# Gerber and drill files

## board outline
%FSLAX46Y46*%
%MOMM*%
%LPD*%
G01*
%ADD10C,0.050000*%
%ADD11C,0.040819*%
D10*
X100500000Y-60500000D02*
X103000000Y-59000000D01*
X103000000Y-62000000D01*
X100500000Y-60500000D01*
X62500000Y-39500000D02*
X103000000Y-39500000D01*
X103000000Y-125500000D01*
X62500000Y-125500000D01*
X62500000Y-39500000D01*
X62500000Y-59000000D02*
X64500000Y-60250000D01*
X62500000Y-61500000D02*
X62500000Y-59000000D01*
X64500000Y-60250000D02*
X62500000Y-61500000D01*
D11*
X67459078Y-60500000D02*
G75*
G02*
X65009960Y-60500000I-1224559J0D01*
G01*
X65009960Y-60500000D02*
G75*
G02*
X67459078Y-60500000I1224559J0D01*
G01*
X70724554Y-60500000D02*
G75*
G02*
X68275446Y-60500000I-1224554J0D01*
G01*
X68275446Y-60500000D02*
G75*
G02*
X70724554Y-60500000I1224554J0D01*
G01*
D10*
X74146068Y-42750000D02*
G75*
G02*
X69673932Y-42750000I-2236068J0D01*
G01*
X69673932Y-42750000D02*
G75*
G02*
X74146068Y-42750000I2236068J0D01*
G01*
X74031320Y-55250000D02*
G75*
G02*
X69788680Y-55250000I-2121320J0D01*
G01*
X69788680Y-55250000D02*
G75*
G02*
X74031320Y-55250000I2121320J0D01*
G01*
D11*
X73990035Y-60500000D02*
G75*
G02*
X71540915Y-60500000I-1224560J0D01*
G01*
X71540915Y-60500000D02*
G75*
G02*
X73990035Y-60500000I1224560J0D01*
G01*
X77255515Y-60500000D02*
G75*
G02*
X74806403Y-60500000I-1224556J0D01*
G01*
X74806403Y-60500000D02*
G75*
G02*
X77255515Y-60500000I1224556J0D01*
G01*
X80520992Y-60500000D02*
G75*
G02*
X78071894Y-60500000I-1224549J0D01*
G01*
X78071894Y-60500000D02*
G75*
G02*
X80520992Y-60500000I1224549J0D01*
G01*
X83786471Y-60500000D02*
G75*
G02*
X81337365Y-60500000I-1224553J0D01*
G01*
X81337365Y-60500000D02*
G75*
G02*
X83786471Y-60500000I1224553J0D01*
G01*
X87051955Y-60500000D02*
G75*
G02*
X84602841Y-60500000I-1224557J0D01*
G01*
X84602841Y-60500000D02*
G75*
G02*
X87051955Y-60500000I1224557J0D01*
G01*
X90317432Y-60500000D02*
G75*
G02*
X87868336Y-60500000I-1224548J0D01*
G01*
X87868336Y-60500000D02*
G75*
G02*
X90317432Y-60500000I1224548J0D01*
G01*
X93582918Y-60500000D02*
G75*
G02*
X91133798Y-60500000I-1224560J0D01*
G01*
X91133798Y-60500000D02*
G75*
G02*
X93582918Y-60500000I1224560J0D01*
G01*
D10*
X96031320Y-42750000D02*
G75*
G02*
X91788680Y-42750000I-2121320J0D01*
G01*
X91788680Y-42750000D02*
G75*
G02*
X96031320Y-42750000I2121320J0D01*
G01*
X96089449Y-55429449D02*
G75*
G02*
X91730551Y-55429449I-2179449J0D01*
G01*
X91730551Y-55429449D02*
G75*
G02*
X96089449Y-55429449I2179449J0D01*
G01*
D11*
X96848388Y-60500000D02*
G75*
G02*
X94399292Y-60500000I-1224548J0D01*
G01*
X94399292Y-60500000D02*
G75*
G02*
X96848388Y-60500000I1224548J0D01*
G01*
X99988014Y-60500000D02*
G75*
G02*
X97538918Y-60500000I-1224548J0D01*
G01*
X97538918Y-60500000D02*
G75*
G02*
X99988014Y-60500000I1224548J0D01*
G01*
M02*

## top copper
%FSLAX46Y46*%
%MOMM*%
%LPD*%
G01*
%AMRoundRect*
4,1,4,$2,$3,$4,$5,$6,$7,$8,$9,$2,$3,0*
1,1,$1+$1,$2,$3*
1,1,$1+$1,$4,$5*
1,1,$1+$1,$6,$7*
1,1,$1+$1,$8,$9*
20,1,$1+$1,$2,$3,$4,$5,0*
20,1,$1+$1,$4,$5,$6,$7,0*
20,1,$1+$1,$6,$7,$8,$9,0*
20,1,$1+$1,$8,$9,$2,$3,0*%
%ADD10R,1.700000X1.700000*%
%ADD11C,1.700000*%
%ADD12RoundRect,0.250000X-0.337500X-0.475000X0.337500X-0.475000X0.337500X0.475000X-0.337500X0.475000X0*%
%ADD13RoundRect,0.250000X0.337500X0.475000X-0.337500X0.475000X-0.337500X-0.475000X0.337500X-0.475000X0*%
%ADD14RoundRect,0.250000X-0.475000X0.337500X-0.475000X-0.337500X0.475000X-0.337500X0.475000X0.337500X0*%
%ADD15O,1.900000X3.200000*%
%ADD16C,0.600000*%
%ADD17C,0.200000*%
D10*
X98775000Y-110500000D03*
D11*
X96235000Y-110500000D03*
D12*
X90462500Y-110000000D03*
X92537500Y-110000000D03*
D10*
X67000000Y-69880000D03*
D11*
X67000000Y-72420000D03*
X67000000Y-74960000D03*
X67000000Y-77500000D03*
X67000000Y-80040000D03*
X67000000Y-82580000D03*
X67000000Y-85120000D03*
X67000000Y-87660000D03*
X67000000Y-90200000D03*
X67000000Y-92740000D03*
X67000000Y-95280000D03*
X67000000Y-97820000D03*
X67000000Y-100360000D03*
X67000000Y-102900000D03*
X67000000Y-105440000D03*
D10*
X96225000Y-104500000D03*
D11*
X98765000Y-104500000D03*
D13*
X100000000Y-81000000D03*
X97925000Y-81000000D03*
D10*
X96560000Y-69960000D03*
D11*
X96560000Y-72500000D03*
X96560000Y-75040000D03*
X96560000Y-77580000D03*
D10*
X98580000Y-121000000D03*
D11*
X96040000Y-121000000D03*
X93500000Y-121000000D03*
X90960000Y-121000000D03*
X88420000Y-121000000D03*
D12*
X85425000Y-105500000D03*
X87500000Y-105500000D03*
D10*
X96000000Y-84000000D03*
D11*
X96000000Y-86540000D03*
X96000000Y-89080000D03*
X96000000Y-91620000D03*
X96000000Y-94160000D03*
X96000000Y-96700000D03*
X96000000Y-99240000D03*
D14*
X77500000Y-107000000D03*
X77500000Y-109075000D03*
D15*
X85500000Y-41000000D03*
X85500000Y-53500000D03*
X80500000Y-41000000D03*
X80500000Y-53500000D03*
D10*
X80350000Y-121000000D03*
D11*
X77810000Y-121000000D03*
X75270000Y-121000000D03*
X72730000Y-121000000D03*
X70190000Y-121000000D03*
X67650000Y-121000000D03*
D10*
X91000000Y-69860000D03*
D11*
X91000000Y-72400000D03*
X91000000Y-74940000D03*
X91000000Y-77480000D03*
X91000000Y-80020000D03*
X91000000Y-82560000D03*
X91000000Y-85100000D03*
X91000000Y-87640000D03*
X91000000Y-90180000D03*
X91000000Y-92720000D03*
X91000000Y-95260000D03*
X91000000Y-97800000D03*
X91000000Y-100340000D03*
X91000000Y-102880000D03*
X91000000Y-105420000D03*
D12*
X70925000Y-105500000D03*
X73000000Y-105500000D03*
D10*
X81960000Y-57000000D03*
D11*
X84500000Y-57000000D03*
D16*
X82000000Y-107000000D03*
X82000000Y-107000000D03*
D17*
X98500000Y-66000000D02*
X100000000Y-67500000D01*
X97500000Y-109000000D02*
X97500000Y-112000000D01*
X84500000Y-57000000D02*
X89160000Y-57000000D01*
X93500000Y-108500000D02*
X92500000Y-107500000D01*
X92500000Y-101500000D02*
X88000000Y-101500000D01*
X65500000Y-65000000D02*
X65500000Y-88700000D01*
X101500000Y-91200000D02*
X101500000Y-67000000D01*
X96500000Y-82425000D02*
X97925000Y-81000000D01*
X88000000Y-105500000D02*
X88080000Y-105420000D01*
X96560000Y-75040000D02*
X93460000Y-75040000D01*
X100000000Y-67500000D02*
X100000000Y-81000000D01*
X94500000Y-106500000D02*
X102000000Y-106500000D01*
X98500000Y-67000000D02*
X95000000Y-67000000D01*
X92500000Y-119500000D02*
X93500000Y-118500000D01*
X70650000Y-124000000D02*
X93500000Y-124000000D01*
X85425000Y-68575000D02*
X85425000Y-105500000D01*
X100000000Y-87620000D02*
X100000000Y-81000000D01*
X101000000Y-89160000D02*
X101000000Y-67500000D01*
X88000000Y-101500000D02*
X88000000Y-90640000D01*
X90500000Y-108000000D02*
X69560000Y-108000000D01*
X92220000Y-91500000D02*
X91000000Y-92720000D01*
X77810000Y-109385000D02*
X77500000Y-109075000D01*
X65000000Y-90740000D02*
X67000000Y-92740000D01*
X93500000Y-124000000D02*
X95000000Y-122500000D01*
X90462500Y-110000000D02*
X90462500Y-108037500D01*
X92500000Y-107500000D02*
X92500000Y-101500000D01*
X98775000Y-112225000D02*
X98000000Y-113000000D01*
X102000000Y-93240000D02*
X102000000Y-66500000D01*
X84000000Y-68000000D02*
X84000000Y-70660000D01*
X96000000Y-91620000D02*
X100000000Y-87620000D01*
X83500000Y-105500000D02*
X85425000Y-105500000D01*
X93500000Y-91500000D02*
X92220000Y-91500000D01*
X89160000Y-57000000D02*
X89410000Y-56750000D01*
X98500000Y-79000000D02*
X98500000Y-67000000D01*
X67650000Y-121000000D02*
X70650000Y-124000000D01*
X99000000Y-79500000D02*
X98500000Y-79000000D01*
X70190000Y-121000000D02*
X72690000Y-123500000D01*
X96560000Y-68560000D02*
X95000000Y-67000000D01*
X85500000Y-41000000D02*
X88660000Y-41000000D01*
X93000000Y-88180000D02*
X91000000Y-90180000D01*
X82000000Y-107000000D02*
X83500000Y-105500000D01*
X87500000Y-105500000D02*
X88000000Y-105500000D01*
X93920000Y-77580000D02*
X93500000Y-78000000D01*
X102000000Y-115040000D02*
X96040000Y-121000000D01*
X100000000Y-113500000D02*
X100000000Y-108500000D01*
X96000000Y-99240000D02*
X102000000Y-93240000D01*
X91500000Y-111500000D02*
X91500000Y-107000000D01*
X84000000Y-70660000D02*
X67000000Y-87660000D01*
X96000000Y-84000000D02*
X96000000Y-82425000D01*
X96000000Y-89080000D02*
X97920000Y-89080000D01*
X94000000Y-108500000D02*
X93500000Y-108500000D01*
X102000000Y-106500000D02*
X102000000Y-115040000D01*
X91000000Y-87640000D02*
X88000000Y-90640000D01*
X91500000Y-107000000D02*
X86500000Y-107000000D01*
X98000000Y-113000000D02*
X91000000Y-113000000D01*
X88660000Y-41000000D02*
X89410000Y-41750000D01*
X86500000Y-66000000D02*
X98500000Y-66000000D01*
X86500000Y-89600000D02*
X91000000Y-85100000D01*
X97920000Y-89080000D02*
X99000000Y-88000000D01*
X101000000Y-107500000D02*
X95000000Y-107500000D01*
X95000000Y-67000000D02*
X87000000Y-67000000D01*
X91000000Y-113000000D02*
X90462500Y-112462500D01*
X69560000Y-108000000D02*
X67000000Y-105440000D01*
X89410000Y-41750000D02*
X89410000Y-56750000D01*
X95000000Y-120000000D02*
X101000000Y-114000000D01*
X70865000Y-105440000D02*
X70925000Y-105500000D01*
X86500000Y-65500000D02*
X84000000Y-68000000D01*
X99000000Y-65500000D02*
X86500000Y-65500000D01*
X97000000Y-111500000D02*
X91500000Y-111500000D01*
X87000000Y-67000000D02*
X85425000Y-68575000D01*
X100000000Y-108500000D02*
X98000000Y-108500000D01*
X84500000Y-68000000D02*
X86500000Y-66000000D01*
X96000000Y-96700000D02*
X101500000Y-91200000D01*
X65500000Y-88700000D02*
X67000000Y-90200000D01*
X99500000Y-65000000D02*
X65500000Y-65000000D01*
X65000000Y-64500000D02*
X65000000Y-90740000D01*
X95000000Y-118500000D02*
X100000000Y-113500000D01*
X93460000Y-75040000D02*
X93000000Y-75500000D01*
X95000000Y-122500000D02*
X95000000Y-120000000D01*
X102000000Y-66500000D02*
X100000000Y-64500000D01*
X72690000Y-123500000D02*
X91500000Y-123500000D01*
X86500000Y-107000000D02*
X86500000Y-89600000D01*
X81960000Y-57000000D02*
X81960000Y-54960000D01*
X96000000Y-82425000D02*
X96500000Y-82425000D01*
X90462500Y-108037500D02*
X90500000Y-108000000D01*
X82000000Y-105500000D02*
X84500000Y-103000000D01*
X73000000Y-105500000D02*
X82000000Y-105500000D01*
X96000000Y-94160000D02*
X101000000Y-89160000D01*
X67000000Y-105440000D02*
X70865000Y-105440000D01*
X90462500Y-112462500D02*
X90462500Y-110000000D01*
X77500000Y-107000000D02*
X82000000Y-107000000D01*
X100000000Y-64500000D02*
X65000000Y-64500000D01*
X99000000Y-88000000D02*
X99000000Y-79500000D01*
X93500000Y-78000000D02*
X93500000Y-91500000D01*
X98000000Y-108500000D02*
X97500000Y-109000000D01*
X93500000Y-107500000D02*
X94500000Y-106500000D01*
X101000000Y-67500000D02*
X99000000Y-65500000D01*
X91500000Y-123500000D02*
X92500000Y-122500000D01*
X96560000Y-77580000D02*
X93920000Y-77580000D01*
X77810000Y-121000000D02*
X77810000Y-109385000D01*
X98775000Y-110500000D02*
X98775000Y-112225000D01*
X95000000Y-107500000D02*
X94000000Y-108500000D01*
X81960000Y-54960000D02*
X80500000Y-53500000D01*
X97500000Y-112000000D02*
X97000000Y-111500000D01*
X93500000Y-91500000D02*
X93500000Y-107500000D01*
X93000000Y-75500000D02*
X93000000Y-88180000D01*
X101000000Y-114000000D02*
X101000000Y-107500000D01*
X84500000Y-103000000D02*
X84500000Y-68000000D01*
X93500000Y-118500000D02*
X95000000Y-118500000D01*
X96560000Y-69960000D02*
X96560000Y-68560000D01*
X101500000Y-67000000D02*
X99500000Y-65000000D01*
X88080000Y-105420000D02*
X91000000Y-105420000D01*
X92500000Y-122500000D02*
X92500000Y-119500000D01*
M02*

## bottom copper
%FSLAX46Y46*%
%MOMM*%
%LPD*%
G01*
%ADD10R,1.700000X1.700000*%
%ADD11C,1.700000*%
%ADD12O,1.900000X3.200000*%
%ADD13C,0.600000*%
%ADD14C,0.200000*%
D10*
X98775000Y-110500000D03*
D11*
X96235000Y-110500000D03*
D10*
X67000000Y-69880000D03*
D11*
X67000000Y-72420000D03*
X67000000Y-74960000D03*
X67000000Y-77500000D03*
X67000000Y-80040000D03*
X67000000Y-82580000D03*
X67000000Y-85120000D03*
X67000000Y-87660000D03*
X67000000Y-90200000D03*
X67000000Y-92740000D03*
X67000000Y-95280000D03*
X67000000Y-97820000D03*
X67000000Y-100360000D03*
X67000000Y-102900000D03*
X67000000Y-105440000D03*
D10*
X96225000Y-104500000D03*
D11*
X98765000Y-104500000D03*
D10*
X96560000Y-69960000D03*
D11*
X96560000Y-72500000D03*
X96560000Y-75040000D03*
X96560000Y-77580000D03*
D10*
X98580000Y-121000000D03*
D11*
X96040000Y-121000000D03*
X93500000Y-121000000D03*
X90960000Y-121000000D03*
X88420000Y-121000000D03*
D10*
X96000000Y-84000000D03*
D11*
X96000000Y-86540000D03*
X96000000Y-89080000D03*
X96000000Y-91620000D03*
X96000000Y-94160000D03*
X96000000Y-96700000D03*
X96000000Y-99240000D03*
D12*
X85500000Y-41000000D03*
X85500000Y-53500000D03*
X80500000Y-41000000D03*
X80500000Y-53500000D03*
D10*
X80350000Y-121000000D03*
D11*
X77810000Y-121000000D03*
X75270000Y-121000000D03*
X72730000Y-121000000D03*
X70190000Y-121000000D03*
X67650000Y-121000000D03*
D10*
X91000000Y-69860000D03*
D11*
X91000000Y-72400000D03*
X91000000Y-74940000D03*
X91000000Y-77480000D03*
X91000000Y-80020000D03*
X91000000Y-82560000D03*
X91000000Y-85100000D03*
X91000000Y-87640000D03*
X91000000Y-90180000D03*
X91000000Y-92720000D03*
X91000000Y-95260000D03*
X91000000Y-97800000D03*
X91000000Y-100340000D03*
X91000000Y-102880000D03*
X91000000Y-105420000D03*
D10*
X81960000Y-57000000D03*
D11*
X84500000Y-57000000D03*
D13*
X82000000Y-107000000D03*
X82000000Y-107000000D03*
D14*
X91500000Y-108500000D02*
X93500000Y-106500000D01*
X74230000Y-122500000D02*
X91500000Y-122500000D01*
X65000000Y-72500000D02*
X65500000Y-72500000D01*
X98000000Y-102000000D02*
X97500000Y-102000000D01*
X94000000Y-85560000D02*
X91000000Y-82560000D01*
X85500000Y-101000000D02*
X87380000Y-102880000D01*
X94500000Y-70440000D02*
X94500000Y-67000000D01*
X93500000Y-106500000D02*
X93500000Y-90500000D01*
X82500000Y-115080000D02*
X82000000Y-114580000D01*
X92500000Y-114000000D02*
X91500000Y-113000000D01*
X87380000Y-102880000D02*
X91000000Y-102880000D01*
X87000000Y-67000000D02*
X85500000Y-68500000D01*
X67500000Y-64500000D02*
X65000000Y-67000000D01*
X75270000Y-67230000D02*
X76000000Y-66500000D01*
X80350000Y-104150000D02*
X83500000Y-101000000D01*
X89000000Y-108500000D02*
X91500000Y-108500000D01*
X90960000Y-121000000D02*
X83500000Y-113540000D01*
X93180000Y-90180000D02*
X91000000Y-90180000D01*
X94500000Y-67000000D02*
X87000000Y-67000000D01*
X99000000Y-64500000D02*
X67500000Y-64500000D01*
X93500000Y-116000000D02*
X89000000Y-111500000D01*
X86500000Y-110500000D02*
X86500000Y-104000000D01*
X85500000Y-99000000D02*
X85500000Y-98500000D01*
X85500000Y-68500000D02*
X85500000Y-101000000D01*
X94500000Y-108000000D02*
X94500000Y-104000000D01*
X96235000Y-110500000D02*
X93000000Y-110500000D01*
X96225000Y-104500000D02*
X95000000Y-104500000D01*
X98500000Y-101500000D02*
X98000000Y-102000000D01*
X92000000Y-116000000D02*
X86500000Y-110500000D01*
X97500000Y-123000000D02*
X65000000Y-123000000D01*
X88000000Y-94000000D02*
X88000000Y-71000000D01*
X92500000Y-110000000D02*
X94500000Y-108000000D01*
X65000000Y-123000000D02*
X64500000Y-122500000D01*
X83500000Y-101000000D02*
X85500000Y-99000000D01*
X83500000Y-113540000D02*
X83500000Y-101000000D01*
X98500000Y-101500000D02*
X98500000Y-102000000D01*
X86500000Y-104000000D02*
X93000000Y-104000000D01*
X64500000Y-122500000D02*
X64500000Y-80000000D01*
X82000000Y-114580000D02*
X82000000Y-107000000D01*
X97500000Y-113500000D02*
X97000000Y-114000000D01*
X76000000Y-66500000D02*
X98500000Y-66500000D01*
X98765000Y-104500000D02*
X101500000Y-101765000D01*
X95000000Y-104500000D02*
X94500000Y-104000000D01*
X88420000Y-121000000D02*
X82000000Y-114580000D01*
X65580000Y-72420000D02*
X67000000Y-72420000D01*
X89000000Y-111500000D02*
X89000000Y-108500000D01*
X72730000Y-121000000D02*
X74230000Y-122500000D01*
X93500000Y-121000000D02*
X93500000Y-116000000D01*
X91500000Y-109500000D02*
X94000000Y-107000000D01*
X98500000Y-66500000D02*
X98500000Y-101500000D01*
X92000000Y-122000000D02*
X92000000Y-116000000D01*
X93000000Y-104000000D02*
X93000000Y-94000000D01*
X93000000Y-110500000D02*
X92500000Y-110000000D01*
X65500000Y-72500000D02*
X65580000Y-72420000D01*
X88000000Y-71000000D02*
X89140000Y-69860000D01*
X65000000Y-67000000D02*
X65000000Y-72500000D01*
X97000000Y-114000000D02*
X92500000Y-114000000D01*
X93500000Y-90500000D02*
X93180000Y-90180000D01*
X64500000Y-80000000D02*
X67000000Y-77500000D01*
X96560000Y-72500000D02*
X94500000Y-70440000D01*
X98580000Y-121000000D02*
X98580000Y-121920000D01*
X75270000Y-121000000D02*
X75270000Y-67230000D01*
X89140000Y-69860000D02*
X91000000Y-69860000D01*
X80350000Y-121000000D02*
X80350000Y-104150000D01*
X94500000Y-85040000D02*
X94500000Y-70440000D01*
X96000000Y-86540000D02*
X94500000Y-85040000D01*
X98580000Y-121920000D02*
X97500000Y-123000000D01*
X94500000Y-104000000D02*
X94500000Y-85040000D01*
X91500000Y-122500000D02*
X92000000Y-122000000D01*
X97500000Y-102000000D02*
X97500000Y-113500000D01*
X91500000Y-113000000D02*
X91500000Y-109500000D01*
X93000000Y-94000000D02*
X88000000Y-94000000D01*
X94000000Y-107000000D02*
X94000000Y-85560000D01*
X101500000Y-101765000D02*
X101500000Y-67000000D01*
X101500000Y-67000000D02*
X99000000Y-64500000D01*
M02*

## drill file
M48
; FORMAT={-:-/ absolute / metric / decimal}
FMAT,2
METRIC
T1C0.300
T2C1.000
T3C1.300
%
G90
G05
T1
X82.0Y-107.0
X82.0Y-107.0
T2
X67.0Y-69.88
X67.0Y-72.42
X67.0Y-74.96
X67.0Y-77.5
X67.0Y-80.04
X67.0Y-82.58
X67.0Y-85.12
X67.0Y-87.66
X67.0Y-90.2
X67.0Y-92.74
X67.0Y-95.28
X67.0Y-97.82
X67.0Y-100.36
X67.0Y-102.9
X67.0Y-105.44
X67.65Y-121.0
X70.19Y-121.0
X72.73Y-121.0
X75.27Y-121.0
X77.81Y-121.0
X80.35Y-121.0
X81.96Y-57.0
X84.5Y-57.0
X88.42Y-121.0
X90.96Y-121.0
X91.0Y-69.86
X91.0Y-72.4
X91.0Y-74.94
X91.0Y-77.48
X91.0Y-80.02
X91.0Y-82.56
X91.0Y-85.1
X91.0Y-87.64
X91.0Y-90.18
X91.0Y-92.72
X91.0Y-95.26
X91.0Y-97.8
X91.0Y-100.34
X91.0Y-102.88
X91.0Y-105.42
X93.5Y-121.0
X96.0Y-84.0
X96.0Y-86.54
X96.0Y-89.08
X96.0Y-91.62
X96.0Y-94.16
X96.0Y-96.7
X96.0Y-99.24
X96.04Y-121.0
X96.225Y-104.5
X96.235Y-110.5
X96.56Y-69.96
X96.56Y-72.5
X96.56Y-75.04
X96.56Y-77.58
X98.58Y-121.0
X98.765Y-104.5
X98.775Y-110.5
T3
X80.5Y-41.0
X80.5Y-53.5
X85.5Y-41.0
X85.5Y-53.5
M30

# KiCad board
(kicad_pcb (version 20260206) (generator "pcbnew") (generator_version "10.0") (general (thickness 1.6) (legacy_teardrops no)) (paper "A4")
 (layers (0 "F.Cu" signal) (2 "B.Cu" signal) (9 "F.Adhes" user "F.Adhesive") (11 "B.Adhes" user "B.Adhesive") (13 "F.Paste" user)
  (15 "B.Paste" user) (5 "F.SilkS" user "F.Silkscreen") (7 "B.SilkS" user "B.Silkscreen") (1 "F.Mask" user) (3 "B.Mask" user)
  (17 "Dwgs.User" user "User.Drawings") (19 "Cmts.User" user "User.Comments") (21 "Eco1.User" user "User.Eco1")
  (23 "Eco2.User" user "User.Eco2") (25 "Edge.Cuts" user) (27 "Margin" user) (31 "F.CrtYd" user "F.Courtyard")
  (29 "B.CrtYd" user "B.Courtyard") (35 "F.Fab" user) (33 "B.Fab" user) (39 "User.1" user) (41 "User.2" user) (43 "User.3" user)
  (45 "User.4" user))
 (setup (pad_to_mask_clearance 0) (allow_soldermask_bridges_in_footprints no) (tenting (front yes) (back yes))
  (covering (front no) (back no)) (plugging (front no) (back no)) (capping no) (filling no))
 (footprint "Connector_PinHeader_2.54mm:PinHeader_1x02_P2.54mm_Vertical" (layer "F.Cu") (at 98.775 110.5 -90)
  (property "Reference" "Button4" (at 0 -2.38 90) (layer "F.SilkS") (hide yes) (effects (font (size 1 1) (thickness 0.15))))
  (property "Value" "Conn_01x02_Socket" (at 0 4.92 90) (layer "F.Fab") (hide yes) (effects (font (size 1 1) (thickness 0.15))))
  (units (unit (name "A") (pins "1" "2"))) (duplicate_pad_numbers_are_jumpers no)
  (pad "1" thru_hole rect (at 0 0 270) (size 1.7 1.7) (drill 1) (layers "*.Cu" "*.Mask") (remove_unused_layers no))
  (pad "2" thru_hole circle (at 0 2.54 270) (size 1.7 1.7) (drill 1) (layers "*.Cu" "*.Mask") (remove_unused_layers no)))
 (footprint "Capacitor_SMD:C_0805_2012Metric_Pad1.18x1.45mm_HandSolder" (layer "F.Cu") (at 91.5 110)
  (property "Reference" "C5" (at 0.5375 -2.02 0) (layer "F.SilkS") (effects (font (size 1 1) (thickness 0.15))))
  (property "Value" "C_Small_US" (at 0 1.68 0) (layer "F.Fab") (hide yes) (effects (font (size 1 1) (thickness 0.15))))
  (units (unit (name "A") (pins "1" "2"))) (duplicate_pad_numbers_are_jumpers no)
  (pad "1" smd roundrect (at -1.0375 0) (size 1.175 1.45) (layers "F.Cu" "F.Mask" "F.Paste") (roundrect_rratio 0.212766))
  (pad "2" smd roundrect (at 1.0375 0) (size 1.175 1.45) (layers "F.Cu" "F.Mask" "F.Paste") (roundrect_rratio 0.212766)))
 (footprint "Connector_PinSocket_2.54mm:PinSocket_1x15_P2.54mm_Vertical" (layer "F.Cu") (at 67 69.88)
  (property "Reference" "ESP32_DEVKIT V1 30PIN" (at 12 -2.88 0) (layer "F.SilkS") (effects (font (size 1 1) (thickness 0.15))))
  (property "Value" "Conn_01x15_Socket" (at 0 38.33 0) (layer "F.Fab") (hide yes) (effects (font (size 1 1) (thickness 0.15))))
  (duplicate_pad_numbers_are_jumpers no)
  (pad "1" thru_hole rect (at 0 0) (size 1.7 1.7) (drill 1) (layers "*.Cu" "*.Mask") (remove_unused_layers no))
  (pad "2" thru_hole circle (at 0 2.54) (size 1.7 1.7) (drill 1) (layers "*.Cu" "*.Mask") (remove_unused_layers no))
  (pad "3" thru_hole circle (at 0 5.08) (size 1.7 1.7) (drill 1) (layers "*.Cu" "*.Mask") (remove_unused_layers no))
  (pad "4" thru_hole circle (at 0 7.62) (size 1.7 1.7) (drill 1) (layers "*.Cu" "*.Mask") (remove_unused_layers no))
  (pad "5" thru_hole circle (at 0 10.16) (size 1.7 1.7) (drill 1) (layers "*.Cu" "*.Mask") (remove_unused_layers no))
  (pad "6" thru_hole circle (at 0 12.7) (size 1.7 1.7) (drill 1) (layers "*.Cu" "*.Mask") (remove_unused_layers no))
  (pad "7" thru_hole circle (at 0 15.24) (size 1.7 1.7) (drill 1) (layers "*.Cu" "*.Mask") (remove_unused_layers no))
  (pad "8" thru_hole circle (at 0 17.78) (size 1.7 1.7) (drill 1) (layers "*.Cu" "*.Mask") (remove_unused_layers no))
  (pad "9" thru_hole circle (at 0 20.32) (size 1.7 1.7) (drill 1) (layers "*.Cu" "*.Mask") (remove_unused_layers no))
  (pad "10" thru_hole circle (at 0 22.86) (size 1.7 1.7) (drill 1) (layers "*.Cu" "*.Mask") (remove_unused_layers no))
  (pad "11" thru_hole circle (at 0 25.4) (size 1.7 1.7) (drill 1) (layers "*.Cu" "*.Mask") (remove_unused_layers no))
  (pad "12" thru_hole circle (at 0 27.94) (size 1.7 1.7) (drill 1) (layers "*.Cu" "*.Mask") (remove_unused_layers no))
  (pad "13" thru_hole circle (at 0 30.48) (size 1.7 1.7) (drill 1) (layers "*.Cu" "*.Mask") (remove_unused_layers no))
  (pad "14" thru_hole circle (at 0 33.02) (size 1.7 1.7) (drill 1) (layers "*.Cu" "*.Mask") (remove_unused_layers no))
  (pad "15" thru_hole circle (at 0 35.56) (size 1.7 1.7) (drill 1) (layers "*.Cu" "*.Mask") (remove_unused_layers no)))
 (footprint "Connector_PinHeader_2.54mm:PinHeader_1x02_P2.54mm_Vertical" (layer "F.Cu") (at 96.225 104.5 90)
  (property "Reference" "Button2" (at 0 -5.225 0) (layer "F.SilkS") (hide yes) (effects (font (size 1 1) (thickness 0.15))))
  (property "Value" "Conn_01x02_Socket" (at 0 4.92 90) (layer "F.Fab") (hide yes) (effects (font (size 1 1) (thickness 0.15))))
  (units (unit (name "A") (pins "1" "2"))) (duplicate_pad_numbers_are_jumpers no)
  (pad "1" thru_hole rect (at 0 0 90) (size 1.7 1.7) (drill 1) (layers "*.Cu" "*.Mask") (remove_unused_layers no))
  (pad "2" thru_hole circle (at 0 2.54 90) (size 1.7 1.7) (drill 1) (layers "*.Cu" "*.Mask") (remove_unused_layers no)))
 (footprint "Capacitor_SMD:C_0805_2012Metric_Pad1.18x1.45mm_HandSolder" (layer "F.Cu") (at 98.9625 81 180)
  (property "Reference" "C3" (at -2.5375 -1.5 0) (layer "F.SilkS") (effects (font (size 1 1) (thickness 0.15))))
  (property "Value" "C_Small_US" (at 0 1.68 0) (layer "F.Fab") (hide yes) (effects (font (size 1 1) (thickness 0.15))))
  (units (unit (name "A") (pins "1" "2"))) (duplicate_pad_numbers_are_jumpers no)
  (pad "1" smd roundrect (at -1.0375 0 180) (size 1.175 1.45) (layers "F.Cu" "F.Mask" "F.Paste") (roundrect_rratio 0.212766))
  (pad "2" smd roundrect (at 1.0375 0 180) (size 1.175 1.45) (layers "F.Cu" "F.Mask" "F.Paste") (roundrect_rratio 0.212766)))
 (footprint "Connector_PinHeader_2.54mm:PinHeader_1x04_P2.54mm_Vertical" (layer "F.Cu") (at 96.56 69.96)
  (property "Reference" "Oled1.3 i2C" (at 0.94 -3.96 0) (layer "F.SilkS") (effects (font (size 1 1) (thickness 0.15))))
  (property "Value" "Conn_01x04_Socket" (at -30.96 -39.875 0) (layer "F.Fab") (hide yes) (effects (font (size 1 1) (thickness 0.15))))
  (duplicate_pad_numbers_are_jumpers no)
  (pad "1" thru_hole rect (at 0 0) (size 1.7 1.7) (drill 1) (layers "*.Cu" "*.Mask") (remove_unused_layers no))
  (pad "2" thru_hole circle (at 0 2.54) (size 1.7 1.7) (drill 1) (layers "*.Cu" "*.Mask") (remove_unused_layers no))
  (pad "3" thru_hole circle (at 0 5.08) (size 1.7 1.7) (drill 1) (layers "*.Cu" "*.Mask") (remove_unused_layers no))
  (pad "4" thru_hole circle (at 0 7.62) (size 1.7 1.7) (drill 1) (layers "*.Cu" "*.Mask") (remove_unused_layers no)))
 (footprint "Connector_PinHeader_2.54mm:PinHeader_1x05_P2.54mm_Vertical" (layer "F.Cu") (at 98.58 121 -90)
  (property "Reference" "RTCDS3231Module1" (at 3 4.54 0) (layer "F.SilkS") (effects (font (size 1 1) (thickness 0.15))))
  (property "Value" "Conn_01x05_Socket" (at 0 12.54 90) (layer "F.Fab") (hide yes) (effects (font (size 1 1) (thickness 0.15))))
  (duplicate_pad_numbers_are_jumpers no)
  (pad "1" thru_hole rect (at 0 0 270) (size 1.7 1.7) (drill 1) (layers "*.Cu" "*.Mask") (remove_unused_layers no))
  (pad "2" thru_hole circle (at 0 2.54 270) (size 1.7 1.7) (drill 1) (layers "*.Cu" "*.Mask") (remove_unused_layers no))
  (pad "3" thru_hole circle (at 0 5.08 270) (size 1.7 1.7) (drill 1) (layers "*.Cu" "*.Mask") (remove_unused_layers no))
  (pad "4" thru_hole circle (at 0 7.62 270) (size 1.7 1.7) (drill 1) (layers "*.Cu" "*.Mask") (remove_unused_layers no))
  (pad "5" thru_hole circle (at 0 10.16 270) (size 1.7 1.7) (drill 1) (layers "*.Cu" "*.Mask") (remove_unused_layers no)))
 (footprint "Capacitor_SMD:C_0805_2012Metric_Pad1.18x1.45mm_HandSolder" (layer "F.Cu") (at 86.4625 105.5)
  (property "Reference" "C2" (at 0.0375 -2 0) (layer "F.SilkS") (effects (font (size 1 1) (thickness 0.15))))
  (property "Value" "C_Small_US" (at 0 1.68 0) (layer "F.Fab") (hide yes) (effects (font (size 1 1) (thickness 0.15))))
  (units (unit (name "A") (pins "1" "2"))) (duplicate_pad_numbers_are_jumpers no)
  (pad "1" smd roundrect (at -1.0375 0) (size 1.175 1.45) (layers "F.Cu" "F.Mask" "F.Paste") (roundrect_rratio 0.212766))
  (pad "2" smd roundrect (at 1.0375 0) (size 1.175 1.45) (layers "F.Cu" "F.Mask" "F.Paste") (roundrect_rratio 0.212766)))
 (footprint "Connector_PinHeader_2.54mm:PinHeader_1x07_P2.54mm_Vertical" (layer "F.Cu") (at 96 84)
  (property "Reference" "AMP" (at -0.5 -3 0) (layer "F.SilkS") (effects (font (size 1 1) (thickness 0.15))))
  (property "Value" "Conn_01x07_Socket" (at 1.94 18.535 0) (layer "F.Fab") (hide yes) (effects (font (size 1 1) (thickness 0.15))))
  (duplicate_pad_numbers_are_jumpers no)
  (pad "1" thru_hole rect (at 0 0) (size 1.7 1.7) (drill 1) (layers "*.Cu" "*.Mask") (remove_unused_layers no))
  (pad "2" thru_hole circle (at 0 2.54) (size 1.7 1.7) (drill 1) (layers "*.Cu" "*.Mask") (remove_unused_layers no))
  (pad "3" thru_hole circle (at 0 5.08) (size 1.7 1.7) (drill 1) (layers "*.Cu" "*.Mask") (remove_unused_layers no))
  (pad "4" thru_hole circle (at 0 7.62) (size 1.7 1.7) (drill 1) (layers "*.Cu" "*.Mask") (remove_unused_layers no))
  (pad "5" thru_hole circle (at 0 10.16) (size 1.7 1.7) (drill 1) (layers "*.Cu" "*.Mask") (remove_unused_layers no))
  (pad "6" thru_hole circle (at 0 12.7) (size 1.7 1.7) (drill 1) (layers "*.Cu" "*.Mask") (remove_unused_layers no))
  (pad "7" thru_hole circle (at 0 15.24) (size 1.7 1.7) (drill 1) (layers "*.Cu" "*.Mask") (remove_unused_layers no)))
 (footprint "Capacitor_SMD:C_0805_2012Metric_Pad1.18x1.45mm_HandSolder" (layer "F.Cu") (at 77.5 108.0375 -90)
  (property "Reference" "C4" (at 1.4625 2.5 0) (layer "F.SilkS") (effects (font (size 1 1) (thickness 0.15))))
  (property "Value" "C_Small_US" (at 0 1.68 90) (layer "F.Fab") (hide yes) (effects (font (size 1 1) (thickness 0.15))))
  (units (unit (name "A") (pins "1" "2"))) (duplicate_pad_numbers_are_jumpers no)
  (pad "1" smd roundrect (at -1.0375 0 270) (size 1.175 1.45) (layers "F.Cu" "F.Mask" "F.Paste") (roundrect_rratio 0.212766))
  (pad "2" smd roundrect (at 1.0375 0 270) (size 1.175 1.45) (layers "F.Cu" "F.Mask" "F.Paste") (roundrect_rratio 0.212766)))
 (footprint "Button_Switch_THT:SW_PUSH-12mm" (layer "F.Cu") (at 85.5 41 -90)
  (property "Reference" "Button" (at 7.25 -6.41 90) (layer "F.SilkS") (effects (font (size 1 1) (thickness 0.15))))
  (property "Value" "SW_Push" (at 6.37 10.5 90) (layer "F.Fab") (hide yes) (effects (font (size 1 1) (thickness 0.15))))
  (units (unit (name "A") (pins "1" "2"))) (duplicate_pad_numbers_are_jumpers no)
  (pad "1" thru_hole oval (at 0 0 270) (size 3.2 1.9) (drill 1.3) (layers "*.Cu" "*.Mask") (remove_unused_layers no))
  (pad "1" thru_hole oval (at 12.5 0 270) (size 3.2 1.9) (drill 1.3) (layers "*.Cu" "*.Mask") (remove_unused_layers no))
  (pad "2" thru_hole oval (at 0 5 270) (size 3.2 1.9) (drill 1.3) (layers "*.Cu" "*.Mask") (remove_unused_layers no))
  (pad "2" thru_hole oval (at 12.5 5 270) (size 3.2 1.9) (drill 1.3) (layers "*.Cu" "*.Mask") (remove_unused_layers no)))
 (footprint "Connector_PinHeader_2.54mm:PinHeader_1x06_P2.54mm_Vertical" (layer "F.Cu") (at 80.35 121 -90)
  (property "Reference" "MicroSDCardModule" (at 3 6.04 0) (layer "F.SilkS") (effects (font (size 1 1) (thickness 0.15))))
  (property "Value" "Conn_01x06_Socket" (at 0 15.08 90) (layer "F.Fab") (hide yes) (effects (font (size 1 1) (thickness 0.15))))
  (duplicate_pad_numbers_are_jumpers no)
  (pad "1" thru_hole rect (at 0 0 270) (size 1.7 1.7) (drill 1) (layers "*.Cu" "*.Mask") (remove_unused_layers no))
  (pad "2" thru_hole circle (at 0 2.54 270) (size 1.7 1.7) (drill 1) (layers "*.Cu" "*.Mask") (remove_unused_layers no))
  (pad "3" thru_hole circle (at 0 5.08 270) (size 1.7 1.7) (drill 1) (layers "*.Cu" "*.Mask") (remove_unused_layers no))
  (pad "4" thru_hole circle (at 0 7.62 270) (size 1.7 1.7) (drill 1) (layers "*.Cu" "*.Mask") (remove_unused_layers no))
  (pad "5" thru_hole circle (at 0 10.16 270) (size 1.7 1.7) (drill 1) (layers "*.Cu" "*.Mask") (remove_unused_layers no))
  (pad "6" thru_hole circle (at 0 12.7 270) (size 1.7 1.7) (drill 1) (layers "*.Cu" "*.Mask") (remove_unused_layers no)))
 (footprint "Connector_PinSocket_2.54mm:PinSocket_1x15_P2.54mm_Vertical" (layer "F.Cu") (at 91 69.86)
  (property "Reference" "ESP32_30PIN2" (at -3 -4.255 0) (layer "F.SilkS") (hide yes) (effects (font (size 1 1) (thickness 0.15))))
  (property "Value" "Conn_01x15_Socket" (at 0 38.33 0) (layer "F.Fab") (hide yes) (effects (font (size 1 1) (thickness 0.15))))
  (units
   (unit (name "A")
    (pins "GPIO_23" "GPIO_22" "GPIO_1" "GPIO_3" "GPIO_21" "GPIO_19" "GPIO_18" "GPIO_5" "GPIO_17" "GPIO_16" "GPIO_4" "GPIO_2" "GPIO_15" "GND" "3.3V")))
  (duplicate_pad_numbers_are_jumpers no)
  (pad "1" thru_hole rect (at 0 0) (size 1.7 1.7) (drill 1) (layers "*.Cu" "*.Mask") (remove_unused_layers no))
  (pad "2" thru_hole circle (at 0 2.54) (size 1.7 1.7) (drill 1) (layers "*.Cu" "*.Mask") (remove_unused_layers no))
  (pad "3" thru_hole circle (at 0 5.08) (size 1.7 1.7) (drill 1) (layers "*.Cu" "*.Mask") (remove_unused_layers no))
  (pad "4" thru_hole circle (at 0 7.62) (size 1.7 1.7) (drill 1) (layers "*.Cu" "*.Mask") (remove_unused_layers no))
  (pad "5" thru_hole circle (at 0 10.16) (size 1.7 1.7) (drill 1) (layers "*.Cu" "*.Mask") (remove_unused_layers no))
  (pad "6" thru_hole circle (at 0 12.7) (size 1.7 1.7) (drill 1) (layers "*.Cu" "*.Mask") (remove_unused_layers no))
  (pad "7" thru_hole circle (at 0 15.24) (size 1.7 1.7) (drill 1) (layers "*.Cu" "*.Mask") (remove_unused_layers no))
  (pad "8" thru_hole circle (at 0 17.78) (size 1.7 1.7) (drill 1) (layers "*.Cu" "*.Mask") (remove_unused_layers no))
  (pad "9" thru_hole circle (at 0 20.32) (size 1.7 1.7) (drill 1) (layers "*.Cu" "*.Mask") (remove_unused_layers no))
  (pad "10" thru_hole circle (at 0 22.86) (size 1.7 1.7) (drill 1) (layers "*.Cu" "*.Mask") (remove_unused_layers no))
  (pad "11" thru_hole circle (at 0 25.4) (size 1.7 1.7) (drill 1) (layers "*.Cu" "*.Mask") (remove_unused_layers no))
  (pad "12" thru_hole circle (at 0 27.94) (size 1.7 1.7) (drill 1) (layers "*.Cu" "*.Mask") (remove_unused_layers no))
  (pad "13" thru_hole circle (at 0 30.48) (size 1.7 1.7) (drill 1) (layers "*.Cu" "*.Mask") (remove_unused_layers no))
  (pad "14" thru_hole circle (at 0 33.02) (size 1.7 1.7) (drill 1) (layers "*.Cu" "*.Mask") (remove_unused_layers no))
  (pad "15" thru_hole circle (at 0 35.56) (size 1.7 1.7) (drill 1) (layers "*.Cu" "*.Mask") (remove_unused_layers no)))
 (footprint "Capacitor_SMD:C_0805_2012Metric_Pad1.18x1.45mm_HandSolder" (layer "F.Cu") (at 71.9625 105.5)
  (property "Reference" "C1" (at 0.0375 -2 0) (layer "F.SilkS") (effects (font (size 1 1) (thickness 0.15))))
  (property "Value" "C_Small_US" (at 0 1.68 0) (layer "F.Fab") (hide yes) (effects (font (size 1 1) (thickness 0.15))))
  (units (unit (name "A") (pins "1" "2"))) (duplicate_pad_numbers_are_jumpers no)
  (pad "1" smd roundrect (at -1.0375 0) (size 1.175 1.45) (layers "F.Cu" "F.Mask" "F.Paste") (roundrect_rratio 0.212766))
  (pad "2" smd roundrect (at 1.0375 0) (size 1.175 1.45) (layers "F.Cu" "F.Mask" "F.Paste") (roundrect_rratio 0.212766)))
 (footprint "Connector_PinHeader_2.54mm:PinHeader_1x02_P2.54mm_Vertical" (layer "B.Cu") (at 81.96 57 -90)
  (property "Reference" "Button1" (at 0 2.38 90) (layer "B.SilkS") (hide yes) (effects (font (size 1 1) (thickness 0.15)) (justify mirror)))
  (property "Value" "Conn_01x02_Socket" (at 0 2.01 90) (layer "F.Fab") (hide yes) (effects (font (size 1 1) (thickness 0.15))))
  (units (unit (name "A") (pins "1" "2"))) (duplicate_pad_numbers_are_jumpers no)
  (pad "1" thru_hole rect (at 0 0 270) (size 1.7 1.7) (drill 1) (layers "*.Cu" "*.Mask") (remove_unused_layers no))
  (pad "2" thru_hole circle (at 0 -2.54 270) (size 1.7 1.7) (drill 1) (layers "*.Cu" "*.Mask") (remove_unused_layers no)))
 (gr_poly (pts (xy 100.5 60.5) (xy 103 59) (xy 103 62)) (stroke (width 0.05) (type solid)) (fill no) (layer "Edge.Cuts"))
 (gr_rect (start 62.5 39.5) (end 103 125.5) (stroke (width 0.05) (type default)) (fill no) (layer "Edge.Cuts"))
 (gr_line (start 62.5 59) (end 64.5 60.25) (stroke (width 0.05) (type default)) (layer "Edge.Cuts"))
 (gr_line (start 62.5 61.5) (end 62.5 59) (stroke (width 0.05) (type default)) (layer "Edge.Cuts"))
 (gr_line (start 64.5 60.25) (end 62.5 61.5) (stroke (width 0.05) (type default)) (layer "Edge.Cuts"))
 (gr_circle (center 66.234519 60.5) (end 67.459078 60.5) (stroke (width 0.040819) (type default)) (fill no) (layer "Edge.Cuts"))
 (gr_circle (center 69.5 60.5) (end 70.724554 60.5) (stroke (width 0.040819) (type default)) (fill no) (layer "Edge.Cuts"))
 (gr_circle (center 71.91 42.75) (end 73.91 41.75) (stroke (width 0.05) (type default)) (fill no) (layer "Edge.Cuts"))
 (gr_circle (center 71.91 55.25) (end 73.41 53.75) (stroke (width 0.05) (type default)) (fill no) (layer "Edge.Cuts"))
 (gr_circle (center 72.765475 60.5) (end 73.990035 60.5) (stroke (width 0.040819) (type default)) (fill no) (layer "Edge.Cuts"))
 (gr_circle (center 76.030959 60.5) (end 77.255515 60.5) (stroke (width 0.040819) (type default)) (fill no) (layer "Edge.Cuts"))
 (gr_circle (center 79.296443 60.5) (end 80.520992 60.5) (stroke (width 0.040819) (type default)) (fill no) (layer "Edge.Cuts"))
 (gr_circle (center 82.561918 60.5) (end 83.786471 60.5) (stroke (width 0.040819) (type default)) (fill no) (layer "Edge.Cuts"))
 (gr_circle (center 85.827398 60.5) (end 87.051955 60.5) (stroke (width 0.040819) (type default)) (fill no) (layer "Edge.Cuts"))
 (gr_circle (center 89.092884 60.5) (end 90.317432 60.5) (stroke (width 0.040819) (type default)) (fill no) (layer "Edge.Cuts"))
 (gr_circle (center 92.358358 60.5) (end 93.582918 60.5) (stroke (width 0.040819) (type default)) (fill no) (layer "Edge.Cuts"))
 (gr_circle (center 93.91 42.75) (end 95.41 41.25) (stroke (width 0.05) (type default)) (fill no) (layer "Edge.Cuts"))
 (gr_circle (center 93.91 55.429449) (end 96.03132 54.929449) (stroke (width 0.05) (type default)) (fill no) (layer "Edge.Cuts"))
 (gr_circle (center 95.62384 60.5) (end 96.848388 60.5) (stroke (width 0.040819) (type default)) (fill no) (layer "Edge.Cuts"))
 (gr_circle (center 98.763466 60.5) (end 99.988014 60.5) (stroke (width 0.040819) (type default)) (fill no) (layer "Edge.Cuts"))
 (segment (start 98.5 66) (end 100 67.5) (width 0.2) (layer "F.Cu") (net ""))
 (segment (start 97.5 109) (end 97.5 112) (width 0.2) (layer "F.Cu") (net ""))
 (segment (start 84.5 57) (end 89.16 57) (width 0.2) (layer "F.Cu") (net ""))
 (segment (start 93.5 108.5) (end 92.5 107.5) (width 0.2) (layer "F.Cu") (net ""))
 (segment (start 92.5 101.5) (end 88 101.5) (width 0.2) (layer "F.Cu") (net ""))
 (segment (start 65.5 65) (end 65.5 88.7) (width 0.2) (layer "F.Cu") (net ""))
 (segment (start 101.5 91.2) (end 101.5 67) (width 0.2) (layer "F.Cu") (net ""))
 (segment (start 96.5 82.425) (end 97.925 81) (width 0.2) (layer "F.Cu") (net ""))
 (segment (start 88 105.5) (end 88.08 105.42) (width 0.2) (layer "F.Cu") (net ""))
 (segment (start 96.56 75.04) (end 93.46 75.04) (width 0.2) (layer "F.Cu") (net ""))
 (segment (start 100 67.5) (end 100 81) (width 0.2) (layer "F.Cu") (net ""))
 (segment (start 94.5 106.5) (end 102 106.5) (width 0.2) (layer "F.Cu") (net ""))
 (segment (start 98.5 67) (end 95 67) (width 0.2) (layer "F.Cu") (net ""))
 (segment (start 92.5 119.5) (end 93.5 118.5) (width 0.2) (layer "F.Cu") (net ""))
 (segment (start 70.65 124) (end 93.5 124) (width 0.2) (layer "F.Cu") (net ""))
 (segment (start 85.425 68.575) (end 85.425 105.5) (width 0.2) (layer "F.Cu") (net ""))
 (segment (start 100 87.62) (end 100 81) (width 0.2) (layer "F.Cu") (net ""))
 (segment (start 101 89.16) (end 101 67.5) (width 0.2) (layer "F.Cu") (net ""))
 (segment (start 88 101.5) (end 88 90.64) (width 0.2) (layer "F.Cu") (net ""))
 (segment (start 90.5 108) (end 69.56 108) (width 0.2) (layer "F.Cu") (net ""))
 (segment (start 92.22 91.5) (end 91 92.72) (width 0.2) (layer "F.Cu") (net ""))
 (segment (start 77.81 109.385) (end 77.5 109.075) (width 0.2) (layer "F.Cu") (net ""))
 (segment (start 65 90.74) (end 67 92.74) (width 0.2) (layer "F.Cu") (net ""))
 (segment (start 93.5 124) (end 95 122.5) (width 0.2) (layer "F.Cu") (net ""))
 (segment (start 90.4625 110) (end 90.4625 108.0375) (width 0.2) (layer "F.Cu") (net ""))
 (segment (start 92.5 107.5) (end 92.5 101.5) (width 0.2) (layer "F.Cu") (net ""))
 (segment (start 98.775 112.225) (end 98 113) (width 0.2) (layer "F.Cu") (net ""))
 (segment (start 102 93.24) (end 102 66.5) (width 0.2) (layer "F.Cu") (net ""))
 (segment (start 84 68) (end 84 70.66) (width 0.2) (layer "F.Cu") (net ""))
 (segment (start 96 91.62) (end 100 87.62) (width 0.2) (layer "F.Cu") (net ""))
 (segment (start 83.5 105.5) (end 85.425 105.5) (width 0.2) (layer "F.Cu") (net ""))
 (segment (start 93.5 91.5) (end 92.22 91.5) (width 0.2) (layer "F.Cu") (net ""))
 (segment (start 89.16 57) (end 89.41 56.75) (width 0.2) (layer "F.Cu") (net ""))
 (segment (start 98.5 79) (end 98.5 67) (width 0.2) (layer "F.Cu") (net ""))
 (segment (start 67.65 121) (end 70.65 124) (width 0.2) (layer "F.Cu") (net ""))
 (segment (start 99 79.5) (end 98.5 79) (width 0.2) (layer "F.Cu") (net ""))
 (segment (start 70.19 121) (end 72.69 123.5) (width 0.2) (layer "F.Cu") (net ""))
 (segment (start 96.56 68.56) (end 95 67) (width 0.2) (layer "F.Cu") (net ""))
 (segment (start 85.5 41) (end 88.66 41) (width 0.2) (layer "F.Cu") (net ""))
 (segment (start 93 88.18) (end 91 90.18) (width 0.2) (layer "F.Cu") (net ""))
 (segment (start 82 107) (end 83.5 105.5) (width 0.2) (layer "F.Cu") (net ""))
 (segment (start 87.5 105.5) (end 88 105.5) (width 0.2) (layer "F.Cu") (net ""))
 (segment (start 93.92 77.58) (end 93.5 78) (width 0.2) (layer "F.Cu") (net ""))
 (segment (start 102 115.04) (end 96.04 121) (width 0.2) (layer "F.Cu") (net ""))
 (segment (start 100 113.5) (end 100 108.5) (width 0.2) (layer "F.Cu") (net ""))
 (segment (start 96 99.24) (end 102 93.24) (width 0.2) (layer "F.Cu") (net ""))
 (segment (start 91.5 111.5) (end 91.5 107) (width 0.2) (layer "F.Cu") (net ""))
 (segment (start 84 70.66) (end 67 87.66) (width 0.2) (layer "F.Cu") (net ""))
 (segment (start 96 84) (end 96 82.425) (width 0.2) (layer "F.Cu") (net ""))
 (segment (start 96 89.08) (end 97.92 89.08) (width 0.2) (layer "F.Cu") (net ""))
 (segment (start 94 108.5) (end 93.5 108.5) (width 0.2) (layer "F.Cu") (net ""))
 (segment (start 102 106.5) (end 102 115.04) (width 0.2) (layer "F.Cu") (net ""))
 (segment (start 91 87.64) (end 88 90.64) (width 0.2) (layer "F.Cu") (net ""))
 (segment (start 91.5 107) (end 86.5 107) (width 0.2) (layer "F.Cu") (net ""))
 (segment (start 98 113) (end 91 113) (width 0.2) (layer "F.Cu") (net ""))
 (segment (start 88.66 41) (end 89.41 41.75) (width 0.2) (layer "F.Cu") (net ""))
 (segment (start 86.5 66) (end 98.5 66) (width 0.2) (layer "F.Cu") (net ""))
 (segment (start 86.5 89.6) (end 91 85.1) (width 0.2) (layer "F.Cu") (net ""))
 (segment (start 97.92 89.08) (end 99 88) (width 0.2) (layer "F.Cu") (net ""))
 (segment (start 101 107.5) (end 95 107.5) (width 0.2) (layer "F.Cu") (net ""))
 (segment (start 95 67) (end 87 67) (width 0.2) (layer "F.Cu") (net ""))
 (segment (start 91 113) (end 90.4625 112.4625) (width 0.2) (layer "F.Cu") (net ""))
 (segment (start 69.56 108) (end 67 105.44) (width 0.2) (layer "F.Cu") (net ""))
 (segment (start 89.41 41.75) (end 89.41 56.75) (width 0.2) (layer "F.Cu") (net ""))
 (segment (start 95 120) (end 101 114) (width 0.2) (layer "F.Cu") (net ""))
 (segment (start 70.865 105.44) (end 70.925 105.5) (width 0.2) (layer "F.Cu") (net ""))
 (segment (start 86.5 65.5) (end 84 68) (width 0.2) (layer "F.Cu") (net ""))
 (segment (start 99 65.5) (end 86.5 65.5) (width 0.2) (layer "F.Cu") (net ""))
 (segment (start 97 111.5) (end 91.5 111.5) (width 0.2) (layer "F.Cu") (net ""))
 (segment (start 87 67) (end 85.425 68.575) (width 0.2) (layer "F.Cu") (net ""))
 (segment (start 100 108.5) (end 98 108.5) (width 0.2) (layer "F.Cu") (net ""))
 (segment (start 84.5 68) (end 86.5 66) (width 0.2) (layer "F.Cu") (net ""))
 (segment (start 96 96.7) (end 101.5 91.2) (width 0.2) (layer "F.Cu") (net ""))
 (segment (start 65.5 88.7) (end 67 90.2) (width 0.2) (layer "F.Cu") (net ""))
 (segment (start 99.5 65) (end 65.5 65) (width 0.2) (layer "F.Cu") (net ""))
 (segment (start 65 64.5) (end 65 90.74) (width 0.2) (layer "F.Cu") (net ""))
 (segment (start 95 118.5) (end 100 113.5) (width 0.2) (layer "F.Cu") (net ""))
 (segment (start 93.46 75.04) (end 93 75.5) (width 0.2) (layer "F.Cu") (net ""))
 (segment (start 95 122.5) (end 95 120) (width 0.2) (layer "F.Cu") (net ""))
 (segment (start 102 66.5) (end 100 64.5) (width 0.2) (layer "F.Cu") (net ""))
 (segment (start 72.69 123.5) (end 91.5 123.5) (width 0.2) (layer "F.Cu") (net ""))
 (segment (start 86.5 107) (end 86.5 89.6) (width 0.2) (layer "F.Cu") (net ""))
 (segment (start 81.96 57) (end 81.96 54.96) (width 0.2) (layer "F.Cu") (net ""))
 (segment (start 96 82.425) (end 96.5 82.425) (width 0.2) (layer "F.Cu") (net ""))
 (segment (start 90.4625 108.0375) (end 90.5 108) (width 0.2) (layer "F.Cu") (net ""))
 (segment (start 82 105.5) (end 84.5 103) (width 0.2) (layer "F.Cu") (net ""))
 (segment (start 73 105.5) (end 82 105.5) (width 0.2) (layer "F.Cu") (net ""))
 (segment (start 96 94.16) (end 101 89.16) (width 0.2) (layer "F.Cu") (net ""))
 (segment (start 67 105.44) (end 70.865 105.44) (width 0.2) (layer "F.Cu") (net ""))
 (segment (start 90.4625 112.4625) (end 90.4625 110) (width 0.2) (layer "F.Cu") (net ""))
 (segment (start 77.5 107) (end 82 107) (width 0.2) (layer "F.Cu") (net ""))
 (segment (start 100 64.5) (end 65 64.5) (width 0.2) (layer "F.Cu") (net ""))
 (segment (start 99 88) (end 99 79.5) (width 0.2) (layer "F.Cu") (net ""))
 (segment (start 93.5 78) (end 93.5 91.5) (width 0.2) (layer "F.Cu") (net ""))
 (segment (start 98 108.5) (end 97.5 109) (width 0.2) (layer "F.Cu") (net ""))
 (segment (start 93.5 107.5) (end 94.5 106.5) (width 0.2) (layer "F.Cu") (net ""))
 (segment (start 101 67.5) (end 99 65.5) (width 0.2) (layer "F.Cu") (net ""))
 (segment (start 91.5 123.5) (end 92.5 122.5) (width 0.2) (layer "F.Cu") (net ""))
 (segment (start 96.56 77.58) (end 93.92 77.58) (width 0.2) (layer "F.Cu") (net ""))
 (segment (start 77.81 121) (end 77.81 109.385) (width 0.2) (layer "F.Cu") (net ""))
 (segment (start 98.775 110.5) (end 98.775 112.225) (width 0.2) (layer "F.Cu") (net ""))
 (segment (start 95 107.5) (end 94 108.5) (width 0.2) (layer "F.Cu") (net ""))
 (segment (start 81.96 54.96) (end 80.5 53.5) (width 0.2) (layer "F.Cu") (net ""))
 (segment (start 97.5 112) (end 97 111.5) (width 0.2) (layer "F.Cu") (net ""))
 (segment (start 93.5 91.5) (end 93.5 107.5) (width 0.2) (layer "F.Cu") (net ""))
 (segment (start 93 75.5) (end 93 88.18) (width 0.2) (layer "F.Cu") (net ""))
 (segment (start 101 114) (end 101 107.5) (width 0.2) (layer "F.Cu") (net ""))
 (segment (start 84.5 103) (end 84.5 68) (width 0.2) (layer "F.Cu") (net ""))
 (segment (start 93.5 118.5) (end 95 118.5) (width 0.2) (layer "F.Cu") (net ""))
 (segment (start 96.56 69.96) (end 96.56 68.56) (width 0.2) (layer "F.Cu") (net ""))
 (segment (start 101.5 67) (end 99.5 65) (width 0.2) (layer "F.Cu") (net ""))
 (segment (start 88.08 105.42) (end 91 105.42) (width 0.2) (layer "F.Cu") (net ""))
 (segment (start 92.5 122.5) (end 92.5 119.5) (width 0.2) (layer "F.Cu") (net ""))
 (via (at 82 107) (size 0.6) (drill 0.3) (layers "F.Cu" "B.Cu") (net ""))
 (via (at 82 107) (size 0.6) (drill 0.3) (layers "F.Cu" "B.Cu") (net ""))
 (segment (start 91.5 108.5) (end 93.5 106.5) (width 0.2) (layer "B.Cu") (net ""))
 (segment (start 74.23 122.5) (end 91.5 122.5) (width 0.2) (layer "B.Cu") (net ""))
 (segment (start 65 72.5) (end 65.5 72.5) (width 0.2) (layer "B.Cu") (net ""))
 (segment (start 98 102) (end 97.5 102) (width 0.2) (layer "B.Cu") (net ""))
 (segment (start 94 85.56) (end 91 82.56) (width 0.2) (layer "B.Cu") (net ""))
 (segment (start 85.5 101) (end 87.38 102.88) (width 0.2) (layer "B.Cu") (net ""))
 (segment (start 94.5 70.44) (end 94.5 67) (width 0.2) (layer "B.Cu") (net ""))
 (segment (start 93.5 106.5) (end 93.5 90.5) (width 0.2) (layer "B.Cu") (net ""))
 (segment (start 82.5 115.08) (end 82 114.58) (width 0.2) (layer "B.Cu") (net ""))
 (segment (start 92.5 114) (end 91.5 113) (width 0.2) (layer "B.Cu") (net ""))
 (segment (start 87.38 102.88) (end 91 102.88) (width 0.2) (layer "B.Cu") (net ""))
 (segment (start 87 67) (end 85.5 68.5) (width 0.2) (layer "B.Cu") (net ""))
 (segment (start 67.5 64.5) (end 65 67) (width 0.2) (layer "B.Cu") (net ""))
 (segment (start 75.27 67.23) (end 76 66.5) (width 0.2) (layer "B.Cu") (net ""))
 (segment (start 80.35 104.15) (end 83.5 101) (width 0.2) (layer "B.Cu") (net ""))
 (segment (start 89 108.5) (end 91.5 108.5) (width 0.2) (layer "B.Cu") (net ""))
 (segment (start 90.96 121) (end 83.5 113.54) (width 0.2) (layer "B.Cu") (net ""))
 (segment (start 93.18 90.18) (end 91 90.18) (width 0.2) (layer "B.Cu") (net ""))
 (segment (start 94.5 67) (end 87 67) (width 0.2) (layer "B.Cu") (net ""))
 (segment (start 99 64.5) (end 67.5 64.5) (width 0.2) (layer "B.Cu") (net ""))
 (segment (start 93.5 116) (end 89 111.5) (width 0.2) (layer "B.Cu") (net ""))
 (segment (start 86.5 110.5) (end 86.5 104) (width 0.2) (layer "B.Cu") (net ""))
 (segment (start 85.5 99) (end 85.5 98.5) (width 0.2) (layer "B.Cu") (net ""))
 (segment (start 85.5 68.5) (end 85.5 101) (width 0.2) (layer "B.Cu") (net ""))
 (segment (start 94.5 108) (end 94.5 104) (width 0.2) (layer "B.Cu") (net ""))
 (segment (start 96.235 110.5) (end 93 110.5) (width 0.2) (layer "B.Cu") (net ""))
 (segment (start 96.225 104.5) (end 95 104.5) (width 0.2) (layer "B.Cu") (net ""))
 (segment (start 98.5 101.5) (end 98 102) (width 0.2) (layer "B.Cu") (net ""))
 (segment (start 92 116) (end 86.5 110.5) (width 0.2) (layer "B.Cu") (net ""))
 (segment (start 97.5 123) (end 65 123) (width 0.2) (layer "B.Cu") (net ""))
 (segment (start 88 94) (end 88 71) (width 0.2) (layer "B.Cu") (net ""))
 (segment (start 92.5 110) (end 94.5 108) (width 0.2) (layer "B.Cu") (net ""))
 (segment (start 65 123) (end 64.5 122.5) (width 0.2) (layer "B.Cu") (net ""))
 (segment (start 83.5 101) (end 85.5 99) (width 0.2) (layer "B.Cu") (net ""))
 (segment (start 83.5 113.54) (end 83.5 101) (width 0.2) (layer "B.Cu") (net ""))
 (segment (start 98.5 101.5) (end 98.5 102) (width 0.2) (layer "B.Cu") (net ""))
 (segment (start 86.5 104) (end 93 104) (width 0.2) (layer "B.Cu") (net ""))
 (segment (start 64.5 122.5) (end 64.5 80) (width 0.2) (layer "B.Cu") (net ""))
 (segment (start 82 114.58) (end 82 107) (width 0.2) (layer "B.Cu") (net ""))
 (segment (start 97.5 113.5) (end 97 114) (width 0.2) (layer "B.Cu") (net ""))
 (segment (start 76 66.5) (end 98.5 66.5) (width 0.2) (layer "B.Cu") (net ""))
 (segment (start 98.765 104.5) (end 101.5 101.765) (width 0.2) (layer "B.Cu") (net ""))
 (segment (start 95 104.5) (end 94.5 104) (width 0.2) (layer "B.Cu") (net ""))
 (segment (start 88.42 121) (end 82 114.58) (width 0.2) (layer "B.Cu") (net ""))
 (segment (start 65.58 72.42) (end 67 72.42) (width 0.2) (layer "B.Cu") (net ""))
 (segment (start 89 111.5) (end 89 108.5) (width 0.2) (layer "B.Cu") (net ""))
 (segment (start 72.73 121) (end 74.23 122.5) (width 0.2) (layer "B.Cu") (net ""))
 (segment (start 93.5 121) (end 93.5 116) (width 0.2) (layer "B.Cu") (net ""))
 (segment (start 91.5 109.5) (end 94 107) (width 0.2) (layer "B.Cu") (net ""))
 (segment (start 98.5 66.5) (end 98.5 101.5) (width 0.2) (layer "B.Cu") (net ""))
 (segment (start 92 122) (end 92 116) (width 0.2) (layer "B.Cu") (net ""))
 (segment (start 93 104) (end 93 94) (width 0.2) (layer "B.Cu") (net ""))
 (segment (start 93 110.5) (end 92.5 110) (width 0.2) (layer "B.Cu") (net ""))
 (segment (start 65.5 72.5) (end 65.58 72.42) (width 0.2) (layer "B.Cu") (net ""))
 (segment (start 88 71) (end 89.14 69.86) (width 0.2) (layer "B.Cu") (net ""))
 (segment (start 65 67) (end 65 72.5) (width 0.2) (layer "B.Cu") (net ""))
 (segment (start 97 114) (end 92.5 114) (width 0.2) (layer "B.Cu") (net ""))
 (segment (start 93.5 90.5) (end 93.18 90.18) (width 0.2) (layer "B.Cu") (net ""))
 (segment (start 64.5 80) (end 67 77.5) (width 0.2) (layer "B.Cu") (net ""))
 (segment (start 96.56 72.5) (end 94.5 70.44) (width 0.2) (layer "B.Cu") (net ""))
 (segment (start 98.58 121) (end 98.58 121.92) (width 0.2) (layer "B.Cu") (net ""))
 (segment (start 75.27 121) (end 75.27 67.23) (width 0.2) (layer "B.Cu") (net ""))
 (segment (start 89.14 69.86) (end 91 69.86) (width 0.2) (layer "B.Cu") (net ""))
 (segment (start 80.35 121) (end 80.35 104.15) (width 0.2) (layer "B.Cu") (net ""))
 (segment (start 94.5 85.04) (end 94.5 70.44) (width 0.2) (layer "B.Cu") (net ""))
 (segment (start 96 86.54) (end 94.5 85.04) (width 0.2) (layer "B.Cu") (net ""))
 (segment (start 98.58 121.92) (end 97.5 123) (width 0.2) (layer "B.Cu") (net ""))
 (segment (start 94.5 104) (end 94.5 85.04) (width 0.2) (layer "B.Cu") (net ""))
 (segment (start 91.5 122.5) (end 92 122) (width 0.2) (layer "B.Cu") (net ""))
 (segment (start 97.5 102) (end 97.5 113.5) (width 0.2) (layer "B.Cu") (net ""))
 (segment (start 91.5 113) (end 91.5 109.5) (width 0.2) (layer "B.Cu") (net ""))
 (segment (start 93 94) (end 88 94) (width 0.2) (layer "B.Cu") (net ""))
 (segment (start 94 107) (end 94 85.56) (width 0.2) (layer "B.Cu") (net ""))
 (segment (start 101.5 101.765) (end 101.5 67) (width 0.2) (layer "B.Cu") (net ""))
 (segment (start 101.5 67) (end 99 64.5) (width 0.2) (layer "B.Cu") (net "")))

